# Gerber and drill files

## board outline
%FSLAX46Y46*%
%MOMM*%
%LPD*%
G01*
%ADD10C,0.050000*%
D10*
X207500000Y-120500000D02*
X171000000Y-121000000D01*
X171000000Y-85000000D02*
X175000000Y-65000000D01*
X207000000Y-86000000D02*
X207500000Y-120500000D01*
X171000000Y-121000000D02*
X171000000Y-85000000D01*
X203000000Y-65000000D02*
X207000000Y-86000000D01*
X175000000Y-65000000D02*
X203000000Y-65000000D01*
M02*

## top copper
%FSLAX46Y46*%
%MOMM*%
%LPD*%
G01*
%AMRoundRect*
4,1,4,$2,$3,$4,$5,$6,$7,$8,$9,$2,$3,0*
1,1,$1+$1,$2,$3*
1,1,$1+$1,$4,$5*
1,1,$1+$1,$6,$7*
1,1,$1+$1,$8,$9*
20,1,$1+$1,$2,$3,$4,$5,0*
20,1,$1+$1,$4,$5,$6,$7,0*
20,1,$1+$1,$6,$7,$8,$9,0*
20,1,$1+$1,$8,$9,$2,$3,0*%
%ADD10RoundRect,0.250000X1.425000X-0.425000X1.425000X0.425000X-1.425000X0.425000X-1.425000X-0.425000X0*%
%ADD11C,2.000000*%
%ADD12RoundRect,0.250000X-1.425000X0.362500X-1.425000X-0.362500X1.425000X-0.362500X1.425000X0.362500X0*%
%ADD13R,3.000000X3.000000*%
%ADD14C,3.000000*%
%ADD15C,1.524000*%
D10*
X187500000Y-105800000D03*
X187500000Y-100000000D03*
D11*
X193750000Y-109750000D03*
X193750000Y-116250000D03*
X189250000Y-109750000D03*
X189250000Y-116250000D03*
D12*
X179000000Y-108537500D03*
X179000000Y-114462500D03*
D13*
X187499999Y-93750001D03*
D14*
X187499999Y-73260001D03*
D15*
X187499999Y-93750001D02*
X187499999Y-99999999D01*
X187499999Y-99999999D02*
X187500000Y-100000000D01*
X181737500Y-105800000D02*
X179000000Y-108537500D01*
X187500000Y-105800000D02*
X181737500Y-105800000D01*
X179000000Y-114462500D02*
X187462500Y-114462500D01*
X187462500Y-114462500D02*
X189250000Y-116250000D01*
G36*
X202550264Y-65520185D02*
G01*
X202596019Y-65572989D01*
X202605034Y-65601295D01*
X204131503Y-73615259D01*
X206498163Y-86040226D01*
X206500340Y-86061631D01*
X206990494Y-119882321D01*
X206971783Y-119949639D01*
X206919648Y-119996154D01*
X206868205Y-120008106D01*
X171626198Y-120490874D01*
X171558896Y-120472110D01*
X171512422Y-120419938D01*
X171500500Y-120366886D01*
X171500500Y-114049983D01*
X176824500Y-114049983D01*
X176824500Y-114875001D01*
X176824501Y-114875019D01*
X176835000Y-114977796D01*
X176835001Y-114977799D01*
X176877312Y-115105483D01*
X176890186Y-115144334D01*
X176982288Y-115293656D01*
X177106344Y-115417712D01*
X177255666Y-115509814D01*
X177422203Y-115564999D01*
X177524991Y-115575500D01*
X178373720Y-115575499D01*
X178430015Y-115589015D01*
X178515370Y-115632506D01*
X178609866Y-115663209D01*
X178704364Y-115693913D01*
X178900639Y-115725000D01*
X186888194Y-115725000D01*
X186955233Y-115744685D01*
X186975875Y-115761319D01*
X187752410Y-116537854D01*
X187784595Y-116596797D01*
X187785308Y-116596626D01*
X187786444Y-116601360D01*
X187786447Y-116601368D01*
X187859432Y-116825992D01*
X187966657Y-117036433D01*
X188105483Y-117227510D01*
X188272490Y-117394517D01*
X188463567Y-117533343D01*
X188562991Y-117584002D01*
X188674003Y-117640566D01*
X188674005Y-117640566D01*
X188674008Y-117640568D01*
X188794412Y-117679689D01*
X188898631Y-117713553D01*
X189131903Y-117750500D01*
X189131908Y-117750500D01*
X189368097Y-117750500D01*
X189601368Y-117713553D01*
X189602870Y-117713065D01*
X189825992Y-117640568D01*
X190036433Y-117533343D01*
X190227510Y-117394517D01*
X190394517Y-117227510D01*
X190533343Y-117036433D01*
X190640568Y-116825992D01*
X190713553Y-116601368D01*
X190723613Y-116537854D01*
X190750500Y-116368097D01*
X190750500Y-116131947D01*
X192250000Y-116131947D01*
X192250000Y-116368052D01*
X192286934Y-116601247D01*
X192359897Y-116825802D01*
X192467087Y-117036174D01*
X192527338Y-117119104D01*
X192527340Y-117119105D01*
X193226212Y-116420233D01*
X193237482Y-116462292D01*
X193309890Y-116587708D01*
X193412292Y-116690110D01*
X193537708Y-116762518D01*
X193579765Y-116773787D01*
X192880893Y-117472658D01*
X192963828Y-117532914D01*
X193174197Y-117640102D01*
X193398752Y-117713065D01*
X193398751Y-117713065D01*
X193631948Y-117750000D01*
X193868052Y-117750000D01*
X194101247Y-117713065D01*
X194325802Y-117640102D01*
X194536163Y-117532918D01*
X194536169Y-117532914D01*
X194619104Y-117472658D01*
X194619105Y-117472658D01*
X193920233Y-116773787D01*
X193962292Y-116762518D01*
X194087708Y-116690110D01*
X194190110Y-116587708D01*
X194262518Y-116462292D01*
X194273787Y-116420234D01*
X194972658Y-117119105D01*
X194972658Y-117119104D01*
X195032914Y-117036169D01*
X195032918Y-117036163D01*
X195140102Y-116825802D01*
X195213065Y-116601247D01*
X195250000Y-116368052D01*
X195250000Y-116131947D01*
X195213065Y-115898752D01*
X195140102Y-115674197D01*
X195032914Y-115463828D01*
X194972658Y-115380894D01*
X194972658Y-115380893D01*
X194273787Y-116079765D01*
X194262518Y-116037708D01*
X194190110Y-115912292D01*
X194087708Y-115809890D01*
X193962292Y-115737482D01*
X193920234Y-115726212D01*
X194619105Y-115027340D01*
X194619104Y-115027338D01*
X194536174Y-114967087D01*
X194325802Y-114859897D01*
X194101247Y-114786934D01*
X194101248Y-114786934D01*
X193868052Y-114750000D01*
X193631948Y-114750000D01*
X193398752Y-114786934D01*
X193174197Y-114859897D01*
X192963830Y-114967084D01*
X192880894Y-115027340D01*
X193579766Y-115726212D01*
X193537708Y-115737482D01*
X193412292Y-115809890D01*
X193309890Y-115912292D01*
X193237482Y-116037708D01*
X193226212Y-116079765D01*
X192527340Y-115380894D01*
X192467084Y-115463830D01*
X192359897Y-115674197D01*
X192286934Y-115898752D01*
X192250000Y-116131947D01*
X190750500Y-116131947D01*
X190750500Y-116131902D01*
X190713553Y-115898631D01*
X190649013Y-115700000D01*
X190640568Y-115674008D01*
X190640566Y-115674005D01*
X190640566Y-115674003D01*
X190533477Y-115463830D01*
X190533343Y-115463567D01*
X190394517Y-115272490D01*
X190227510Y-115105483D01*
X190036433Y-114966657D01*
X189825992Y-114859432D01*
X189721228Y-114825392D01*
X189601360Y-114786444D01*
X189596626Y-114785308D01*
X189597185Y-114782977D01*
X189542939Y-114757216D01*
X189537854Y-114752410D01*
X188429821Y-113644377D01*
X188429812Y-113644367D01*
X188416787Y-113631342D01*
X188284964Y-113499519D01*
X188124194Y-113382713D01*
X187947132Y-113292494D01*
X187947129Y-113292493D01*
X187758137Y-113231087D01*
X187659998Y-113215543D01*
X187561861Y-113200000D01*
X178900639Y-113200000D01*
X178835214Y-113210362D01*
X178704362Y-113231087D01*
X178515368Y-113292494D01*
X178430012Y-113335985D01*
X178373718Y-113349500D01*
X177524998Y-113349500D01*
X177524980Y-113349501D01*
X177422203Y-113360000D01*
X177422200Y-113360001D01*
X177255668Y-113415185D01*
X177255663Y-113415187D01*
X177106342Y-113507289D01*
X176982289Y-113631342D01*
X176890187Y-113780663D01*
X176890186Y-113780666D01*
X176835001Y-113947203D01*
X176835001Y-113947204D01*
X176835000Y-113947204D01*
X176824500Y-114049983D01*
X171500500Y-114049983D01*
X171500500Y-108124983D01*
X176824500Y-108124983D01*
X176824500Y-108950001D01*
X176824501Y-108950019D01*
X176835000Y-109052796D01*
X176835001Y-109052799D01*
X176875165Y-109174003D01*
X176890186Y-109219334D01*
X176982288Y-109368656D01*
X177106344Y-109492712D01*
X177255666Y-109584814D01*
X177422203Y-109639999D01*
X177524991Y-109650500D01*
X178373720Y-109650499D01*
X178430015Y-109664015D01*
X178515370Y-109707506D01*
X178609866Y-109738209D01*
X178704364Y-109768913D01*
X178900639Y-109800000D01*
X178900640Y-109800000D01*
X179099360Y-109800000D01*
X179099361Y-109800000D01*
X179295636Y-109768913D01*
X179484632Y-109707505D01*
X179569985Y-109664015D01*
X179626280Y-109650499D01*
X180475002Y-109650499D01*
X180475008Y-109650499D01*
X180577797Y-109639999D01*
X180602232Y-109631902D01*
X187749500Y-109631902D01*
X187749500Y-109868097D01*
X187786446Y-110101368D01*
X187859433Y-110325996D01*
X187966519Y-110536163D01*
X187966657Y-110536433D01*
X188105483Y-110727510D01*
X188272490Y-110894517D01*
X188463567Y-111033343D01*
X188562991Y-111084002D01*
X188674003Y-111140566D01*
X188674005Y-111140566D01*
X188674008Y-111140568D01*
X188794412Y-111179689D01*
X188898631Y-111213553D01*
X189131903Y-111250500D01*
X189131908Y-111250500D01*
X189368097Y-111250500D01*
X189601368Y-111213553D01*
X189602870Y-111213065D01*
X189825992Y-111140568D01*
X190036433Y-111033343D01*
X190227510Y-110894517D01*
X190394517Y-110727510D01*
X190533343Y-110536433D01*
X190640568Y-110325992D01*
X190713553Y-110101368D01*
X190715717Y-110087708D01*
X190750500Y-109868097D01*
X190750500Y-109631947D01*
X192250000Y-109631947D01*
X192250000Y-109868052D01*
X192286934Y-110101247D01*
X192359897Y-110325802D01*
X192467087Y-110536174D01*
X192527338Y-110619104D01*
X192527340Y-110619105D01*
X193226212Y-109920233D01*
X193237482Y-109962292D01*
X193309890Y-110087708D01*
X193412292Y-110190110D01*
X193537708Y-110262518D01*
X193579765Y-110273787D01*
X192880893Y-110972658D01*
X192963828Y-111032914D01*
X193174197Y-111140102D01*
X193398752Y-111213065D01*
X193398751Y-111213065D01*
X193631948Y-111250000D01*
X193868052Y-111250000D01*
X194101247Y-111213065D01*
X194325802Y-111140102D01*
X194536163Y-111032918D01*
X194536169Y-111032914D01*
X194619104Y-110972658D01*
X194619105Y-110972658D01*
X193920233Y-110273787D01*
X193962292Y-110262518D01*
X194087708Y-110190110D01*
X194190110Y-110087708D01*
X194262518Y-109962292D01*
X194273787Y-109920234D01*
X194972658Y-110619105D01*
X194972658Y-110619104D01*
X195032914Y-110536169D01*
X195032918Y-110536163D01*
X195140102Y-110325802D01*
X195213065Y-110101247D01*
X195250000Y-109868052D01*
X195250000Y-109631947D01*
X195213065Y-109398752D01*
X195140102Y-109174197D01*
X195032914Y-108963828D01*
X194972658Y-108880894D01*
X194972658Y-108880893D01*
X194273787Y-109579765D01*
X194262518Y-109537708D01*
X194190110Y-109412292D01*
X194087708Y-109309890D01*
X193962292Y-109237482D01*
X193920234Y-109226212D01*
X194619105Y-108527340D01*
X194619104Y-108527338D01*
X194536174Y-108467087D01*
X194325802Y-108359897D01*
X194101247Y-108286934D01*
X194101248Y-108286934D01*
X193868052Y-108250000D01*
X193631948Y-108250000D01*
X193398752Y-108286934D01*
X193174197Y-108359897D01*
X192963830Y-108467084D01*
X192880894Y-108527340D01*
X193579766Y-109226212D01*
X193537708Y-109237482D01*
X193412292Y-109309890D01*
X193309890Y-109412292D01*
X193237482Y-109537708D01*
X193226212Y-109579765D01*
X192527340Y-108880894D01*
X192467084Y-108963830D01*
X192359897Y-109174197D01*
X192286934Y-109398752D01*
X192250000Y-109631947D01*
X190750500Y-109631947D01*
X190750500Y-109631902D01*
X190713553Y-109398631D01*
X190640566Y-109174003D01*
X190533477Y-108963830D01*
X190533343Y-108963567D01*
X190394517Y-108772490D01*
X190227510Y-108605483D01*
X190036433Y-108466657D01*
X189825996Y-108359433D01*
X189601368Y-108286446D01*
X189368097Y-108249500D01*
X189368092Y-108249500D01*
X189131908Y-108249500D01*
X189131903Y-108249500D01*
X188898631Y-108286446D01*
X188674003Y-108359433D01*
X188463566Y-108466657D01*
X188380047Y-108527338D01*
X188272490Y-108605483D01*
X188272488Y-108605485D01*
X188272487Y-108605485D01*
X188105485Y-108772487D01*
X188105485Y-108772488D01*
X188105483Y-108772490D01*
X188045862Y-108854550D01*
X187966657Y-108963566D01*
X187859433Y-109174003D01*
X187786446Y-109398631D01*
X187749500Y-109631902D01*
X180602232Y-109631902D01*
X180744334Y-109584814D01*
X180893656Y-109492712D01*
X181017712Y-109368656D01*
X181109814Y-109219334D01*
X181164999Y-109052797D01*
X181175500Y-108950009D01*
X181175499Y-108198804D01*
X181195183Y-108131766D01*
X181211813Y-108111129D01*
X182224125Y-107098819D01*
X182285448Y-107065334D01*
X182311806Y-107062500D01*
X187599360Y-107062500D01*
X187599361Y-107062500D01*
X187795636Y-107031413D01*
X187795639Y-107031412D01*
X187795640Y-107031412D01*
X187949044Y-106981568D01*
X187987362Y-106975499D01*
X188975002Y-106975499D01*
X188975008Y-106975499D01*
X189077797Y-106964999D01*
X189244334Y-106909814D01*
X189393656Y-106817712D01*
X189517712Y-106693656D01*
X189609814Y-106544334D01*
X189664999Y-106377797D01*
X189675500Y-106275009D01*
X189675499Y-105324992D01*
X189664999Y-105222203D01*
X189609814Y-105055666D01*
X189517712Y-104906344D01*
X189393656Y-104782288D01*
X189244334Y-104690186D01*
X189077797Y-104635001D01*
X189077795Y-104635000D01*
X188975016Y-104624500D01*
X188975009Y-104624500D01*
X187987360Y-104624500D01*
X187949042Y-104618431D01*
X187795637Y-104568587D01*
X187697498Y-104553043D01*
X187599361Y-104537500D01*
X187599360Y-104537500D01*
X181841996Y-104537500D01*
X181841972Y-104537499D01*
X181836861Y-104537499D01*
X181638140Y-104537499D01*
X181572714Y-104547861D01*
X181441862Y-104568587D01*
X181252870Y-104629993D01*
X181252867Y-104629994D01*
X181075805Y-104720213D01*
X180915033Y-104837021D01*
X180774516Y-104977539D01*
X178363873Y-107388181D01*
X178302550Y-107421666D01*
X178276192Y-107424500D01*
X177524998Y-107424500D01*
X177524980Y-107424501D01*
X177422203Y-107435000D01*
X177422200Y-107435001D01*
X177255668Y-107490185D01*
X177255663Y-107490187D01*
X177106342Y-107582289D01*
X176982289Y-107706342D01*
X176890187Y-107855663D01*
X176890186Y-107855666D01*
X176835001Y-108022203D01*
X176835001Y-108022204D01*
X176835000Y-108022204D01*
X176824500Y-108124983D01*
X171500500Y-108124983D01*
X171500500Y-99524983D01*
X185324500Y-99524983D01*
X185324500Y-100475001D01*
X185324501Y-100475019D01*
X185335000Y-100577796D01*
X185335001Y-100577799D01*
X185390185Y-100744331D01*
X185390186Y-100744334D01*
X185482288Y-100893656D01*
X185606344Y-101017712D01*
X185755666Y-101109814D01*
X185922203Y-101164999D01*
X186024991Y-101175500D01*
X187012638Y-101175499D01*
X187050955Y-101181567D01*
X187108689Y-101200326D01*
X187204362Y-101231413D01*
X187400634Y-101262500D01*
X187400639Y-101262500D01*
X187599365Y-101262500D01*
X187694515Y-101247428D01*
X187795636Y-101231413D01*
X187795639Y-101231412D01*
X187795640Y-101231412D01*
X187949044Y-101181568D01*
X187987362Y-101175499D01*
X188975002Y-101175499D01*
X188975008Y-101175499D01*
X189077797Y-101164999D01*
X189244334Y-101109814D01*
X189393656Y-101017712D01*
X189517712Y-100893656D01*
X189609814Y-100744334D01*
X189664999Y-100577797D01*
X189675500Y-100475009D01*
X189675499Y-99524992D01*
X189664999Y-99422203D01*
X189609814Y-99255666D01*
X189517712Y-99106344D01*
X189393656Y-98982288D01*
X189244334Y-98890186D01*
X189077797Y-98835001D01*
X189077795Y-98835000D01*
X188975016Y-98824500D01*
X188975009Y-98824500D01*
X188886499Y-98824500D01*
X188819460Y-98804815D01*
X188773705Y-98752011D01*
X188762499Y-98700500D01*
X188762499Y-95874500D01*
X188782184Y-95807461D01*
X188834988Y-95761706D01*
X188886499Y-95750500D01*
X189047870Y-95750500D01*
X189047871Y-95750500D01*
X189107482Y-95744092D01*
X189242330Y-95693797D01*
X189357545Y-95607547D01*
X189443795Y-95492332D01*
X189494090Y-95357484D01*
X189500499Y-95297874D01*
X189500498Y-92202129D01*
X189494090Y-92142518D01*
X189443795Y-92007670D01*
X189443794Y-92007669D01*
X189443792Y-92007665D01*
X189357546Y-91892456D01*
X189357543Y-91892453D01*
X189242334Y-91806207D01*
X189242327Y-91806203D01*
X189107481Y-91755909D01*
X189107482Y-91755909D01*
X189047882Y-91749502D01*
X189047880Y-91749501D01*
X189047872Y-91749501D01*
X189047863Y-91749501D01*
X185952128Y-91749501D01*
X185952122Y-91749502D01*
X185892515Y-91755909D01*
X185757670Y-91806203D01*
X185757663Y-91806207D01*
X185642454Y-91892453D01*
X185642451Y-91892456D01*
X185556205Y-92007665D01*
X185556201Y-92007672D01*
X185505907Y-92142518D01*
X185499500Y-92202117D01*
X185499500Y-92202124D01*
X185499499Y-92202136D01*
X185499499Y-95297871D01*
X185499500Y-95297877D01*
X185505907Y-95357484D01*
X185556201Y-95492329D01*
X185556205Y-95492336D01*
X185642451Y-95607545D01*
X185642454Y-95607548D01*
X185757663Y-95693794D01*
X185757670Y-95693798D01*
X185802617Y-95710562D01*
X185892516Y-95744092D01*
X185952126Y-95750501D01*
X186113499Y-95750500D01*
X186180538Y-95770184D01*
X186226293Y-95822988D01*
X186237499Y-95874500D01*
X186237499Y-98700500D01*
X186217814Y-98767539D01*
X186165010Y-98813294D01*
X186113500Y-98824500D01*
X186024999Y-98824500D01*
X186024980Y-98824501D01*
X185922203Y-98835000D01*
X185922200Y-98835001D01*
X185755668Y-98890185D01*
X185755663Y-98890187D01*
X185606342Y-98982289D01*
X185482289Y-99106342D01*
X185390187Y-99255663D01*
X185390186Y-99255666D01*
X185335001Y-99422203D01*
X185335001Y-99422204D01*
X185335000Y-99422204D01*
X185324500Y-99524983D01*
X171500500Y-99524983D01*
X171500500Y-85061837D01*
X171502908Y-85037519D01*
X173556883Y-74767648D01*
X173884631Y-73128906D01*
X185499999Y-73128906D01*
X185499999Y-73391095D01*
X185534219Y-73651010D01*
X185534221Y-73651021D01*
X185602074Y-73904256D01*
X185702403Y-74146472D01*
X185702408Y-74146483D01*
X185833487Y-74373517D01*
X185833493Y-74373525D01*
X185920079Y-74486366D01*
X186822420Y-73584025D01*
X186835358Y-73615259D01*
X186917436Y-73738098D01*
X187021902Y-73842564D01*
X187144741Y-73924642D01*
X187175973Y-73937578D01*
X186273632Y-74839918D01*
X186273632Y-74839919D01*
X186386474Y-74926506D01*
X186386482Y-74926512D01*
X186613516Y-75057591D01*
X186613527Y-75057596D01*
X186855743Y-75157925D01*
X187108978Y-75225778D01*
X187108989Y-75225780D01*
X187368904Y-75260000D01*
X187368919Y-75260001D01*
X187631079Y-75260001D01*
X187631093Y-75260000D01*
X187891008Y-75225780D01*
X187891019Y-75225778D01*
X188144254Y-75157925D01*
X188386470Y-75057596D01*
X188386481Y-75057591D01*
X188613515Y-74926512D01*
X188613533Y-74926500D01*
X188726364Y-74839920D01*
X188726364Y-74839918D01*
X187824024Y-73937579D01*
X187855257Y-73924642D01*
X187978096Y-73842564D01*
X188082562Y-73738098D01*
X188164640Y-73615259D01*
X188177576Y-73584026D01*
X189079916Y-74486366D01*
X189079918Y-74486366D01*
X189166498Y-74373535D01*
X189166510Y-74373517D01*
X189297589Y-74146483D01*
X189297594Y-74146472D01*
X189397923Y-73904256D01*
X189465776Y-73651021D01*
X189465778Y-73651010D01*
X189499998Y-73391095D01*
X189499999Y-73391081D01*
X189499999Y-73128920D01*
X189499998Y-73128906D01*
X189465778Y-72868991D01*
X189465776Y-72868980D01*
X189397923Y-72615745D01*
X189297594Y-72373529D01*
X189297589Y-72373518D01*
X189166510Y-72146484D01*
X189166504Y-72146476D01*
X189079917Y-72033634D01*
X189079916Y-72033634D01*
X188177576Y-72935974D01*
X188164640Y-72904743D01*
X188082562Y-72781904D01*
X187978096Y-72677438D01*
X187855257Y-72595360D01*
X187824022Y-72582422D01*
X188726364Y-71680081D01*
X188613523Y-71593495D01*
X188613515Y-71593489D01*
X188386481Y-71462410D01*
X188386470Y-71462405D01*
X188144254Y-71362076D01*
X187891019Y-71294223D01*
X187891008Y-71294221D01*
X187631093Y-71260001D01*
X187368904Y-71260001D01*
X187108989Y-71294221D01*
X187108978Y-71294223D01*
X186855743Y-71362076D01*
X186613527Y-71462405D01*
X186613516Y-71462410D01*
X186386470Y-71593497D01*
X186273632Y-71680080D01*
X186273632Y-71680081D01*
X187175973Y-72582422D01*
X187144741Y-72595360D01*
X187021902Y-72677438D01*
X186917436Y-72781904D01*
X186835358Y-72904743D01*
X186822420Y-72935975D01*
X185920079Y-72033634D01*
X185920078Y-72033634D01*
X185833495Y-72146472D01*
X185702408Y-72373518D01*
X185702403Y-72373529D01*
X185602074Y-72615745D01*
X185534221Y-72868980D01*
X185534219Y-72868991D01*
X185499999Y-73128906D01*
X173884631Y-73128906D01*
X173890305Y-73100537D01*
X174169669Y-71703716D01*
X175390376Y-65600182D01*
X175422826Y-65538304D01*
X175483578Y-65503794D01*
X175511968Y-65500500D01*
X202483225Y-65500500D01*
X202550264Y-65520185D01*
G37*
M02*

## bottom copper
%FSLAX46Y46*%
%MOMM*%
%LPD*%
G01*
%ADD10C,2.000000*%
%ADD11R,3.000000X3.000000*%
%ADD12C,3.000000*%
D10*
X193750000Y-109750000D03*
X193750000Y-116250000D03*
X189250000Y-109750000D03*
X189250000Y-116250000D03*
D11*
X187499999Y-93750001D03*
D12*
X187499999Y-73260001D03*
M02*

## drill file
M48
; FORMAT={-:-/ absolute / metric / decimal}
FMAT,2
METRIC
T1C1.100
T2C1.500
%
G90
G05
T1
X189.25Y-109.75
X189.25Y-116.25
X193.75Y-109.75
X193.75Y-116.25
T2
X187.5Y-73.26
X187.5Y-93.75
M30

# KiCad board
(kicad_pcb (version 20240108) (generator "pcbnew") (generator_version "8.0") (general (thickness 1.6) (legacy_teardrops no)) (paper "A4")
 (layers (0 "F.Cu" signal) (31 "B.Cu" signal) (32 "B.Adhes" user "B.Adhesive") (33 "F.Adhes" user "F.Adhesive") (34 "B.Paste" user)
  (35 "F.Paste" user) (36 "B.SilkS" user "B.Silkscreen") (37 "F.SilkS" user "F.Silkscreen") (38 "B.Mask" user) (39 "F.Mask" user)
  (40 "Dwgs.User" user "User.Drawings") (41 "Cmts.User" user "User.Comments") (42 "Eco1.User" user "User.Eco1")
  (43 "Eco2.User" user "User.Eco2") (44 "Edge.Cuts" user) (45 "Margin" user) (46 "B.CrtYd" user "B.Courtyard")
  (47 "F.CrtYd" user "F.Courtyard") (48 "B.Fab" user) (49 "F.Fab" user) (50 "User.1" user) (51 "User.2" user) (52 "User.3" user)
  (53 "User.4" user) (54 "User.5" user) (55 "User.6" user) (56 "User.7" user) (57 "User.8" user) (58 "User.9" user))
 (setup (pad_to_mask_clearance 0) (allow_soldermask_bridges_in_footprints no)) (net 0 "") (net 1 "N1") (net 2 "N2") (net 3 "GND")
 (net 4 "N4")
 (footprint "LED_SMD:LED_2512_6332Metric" (layer "F.Cu") (at 187.5 102.9 90)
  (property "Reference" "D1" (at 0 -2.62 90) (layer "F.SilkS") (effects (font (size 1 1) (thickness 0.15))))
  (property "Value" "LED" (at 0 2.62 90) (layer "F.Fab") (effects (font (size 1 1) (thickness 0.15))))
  (pad "1" smd roundrect (at -2.9 0 90) (size 1.35 3.35) (layers "F.Cu" "F.Paste" "F.Mask") (roundrect_rratio 0.185185) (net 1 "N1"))
  (pad "2" smd roundrect (at 2.9 0 90) (size 1.35 3.35) (layers "F.Cu" "F.Paste" "F.Mask") (roundrect_rratio 0.185185) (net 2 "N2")))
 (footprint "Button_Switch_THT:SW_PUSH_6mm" (layer "F.Cu") (at 193.75 109.75 -90)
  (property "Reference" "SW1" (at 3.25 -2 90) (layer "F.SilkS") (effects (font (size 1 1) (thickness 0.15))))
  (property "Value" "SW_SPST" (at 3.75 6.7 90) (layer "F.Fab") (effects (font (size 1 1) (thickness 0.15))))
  (pad "1" thru_hole circle (at 0 0) (size 2 2) (drill 1.1) (layers "*.Cu" "*.Mask") (remove_unused_layers no) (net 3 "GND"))
  (pad "1" thru_hole circle (at 6.5 0) (size 2 2) (drill 1.1) (layers "*.Cu" "*.Mask") (remove_unused_layers no) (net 3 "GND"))
  (pad "2" thru_hole circle (at 0 4.5) (size 2 2) (drill 1.1) (layers "*.Cu" "*.Mask") (remove_unused_layers no) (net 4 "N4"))
  (pad "2" thru_hole circle (at 6.5 4.5) (size 2 2) (drill 1.1) (layers "*.Cu" "*.Mask") (remove_unused_layers no) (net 4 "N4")))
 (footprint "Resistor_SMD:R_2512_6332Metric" (layer "F.Cu") (at 179 111.5 -90)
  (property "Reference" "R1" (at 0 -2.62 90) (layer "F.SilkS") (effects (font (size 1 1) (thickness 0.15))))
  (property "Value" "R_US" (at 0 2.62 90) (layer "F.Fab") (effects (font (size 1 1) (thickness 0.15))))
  (pad "1" smd roundrect (at -2.9625 0 270) (size 1.225 3.35) (layers "F.Cu" "F.Paste" "F.Mask") (roundrect_rratio 0.204082) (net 1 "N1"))
  (pad "2" smd roundrect (at 2.9625 0 270) (size 1.225 3.35) (layers "F.Cu" "F.Paste" "F.Mask") (roundrect_rratio 0.204082) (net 4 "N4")))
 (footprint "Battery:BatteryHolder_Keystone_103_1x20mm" (layer "F.Cu") (at 187.499999 93.750001 90)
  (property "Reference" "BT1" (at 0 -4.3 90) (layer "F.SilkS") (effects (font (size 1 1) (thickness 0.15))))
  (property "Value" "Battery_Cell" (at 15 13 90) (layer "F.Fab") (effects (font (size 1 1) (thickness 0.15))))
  (pad "1" thru_hole rect (at 0 0 90) (size 3 3) (drill 1.5) (layers "*.Cu" "*.Mask") (remove_unused_layers no) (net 2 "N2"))
  (pad "2" thru_hole circle (at 20.49 0 90) (size 3 3) (drill 1.5) (layers "*.Cu" "*.Mask") (remove_unused_layers no) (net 3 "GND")))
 (gr_line (start 207.5 120.5) (end 171 121) (stroke (width 0.05) (type default)) (layer "Edge.Cuts"))
 (gr_line (start 171 85) (end 175 65) (stroke (width 0.05) (type default)) (layer "Edge.Cuts"))
 (gr_line (start 207 86) (end 207.5 120.5) (stroke (width 0.05) (type default)) (layer "Edge.Cuts"))
 (gr_line (start 171 121) (end 171 85) (stroke (width 0.05) (type default)) (layer "Edge.Cuts"))
 (gr_line (start 203 65) (end 207 86) (stroke (width 0.05) (type default)) (layer "Edge.Cuts"))
 (gr_line (start 175 65) (end 203 65) (stroke (width 0.05) (type default)) (layer "Edge.Cuts"))
 (segment (start 187.499999 93.750001) (end 187.499999 99.999999) (width 1.524) (layer "F.Cu") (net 2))
 (segment (start 187.499999 99.999999) (end 187.5 100) (width 1.524) (layer "F.Cu") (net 2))
 (segment (start 181.7375 105.8) (end 179 108.5375) (width 1.524) (layer "F.Cu") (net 1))
 (segment (start 187.5 105.8) (end 181.7375 105.8) (width 1.524) (layer "F.Cu") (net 1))
 (segment (start 179 114.4625) (end 187.4625 114.4625) (width 1.524) (layer "F.Cu") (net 4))
 (segment (start 187.4625 114.4625) (end 189.25 116.25) (width 1.524) (layer "F.Cu") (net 4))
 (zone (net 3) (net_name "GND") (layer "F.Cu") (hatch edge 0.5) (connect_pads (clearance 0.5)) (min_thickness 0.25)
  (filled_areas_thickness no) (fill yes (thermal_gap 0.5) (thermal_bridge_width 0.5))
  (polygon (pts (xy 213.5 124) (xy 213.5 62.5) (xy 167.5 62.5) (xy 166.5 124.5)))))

